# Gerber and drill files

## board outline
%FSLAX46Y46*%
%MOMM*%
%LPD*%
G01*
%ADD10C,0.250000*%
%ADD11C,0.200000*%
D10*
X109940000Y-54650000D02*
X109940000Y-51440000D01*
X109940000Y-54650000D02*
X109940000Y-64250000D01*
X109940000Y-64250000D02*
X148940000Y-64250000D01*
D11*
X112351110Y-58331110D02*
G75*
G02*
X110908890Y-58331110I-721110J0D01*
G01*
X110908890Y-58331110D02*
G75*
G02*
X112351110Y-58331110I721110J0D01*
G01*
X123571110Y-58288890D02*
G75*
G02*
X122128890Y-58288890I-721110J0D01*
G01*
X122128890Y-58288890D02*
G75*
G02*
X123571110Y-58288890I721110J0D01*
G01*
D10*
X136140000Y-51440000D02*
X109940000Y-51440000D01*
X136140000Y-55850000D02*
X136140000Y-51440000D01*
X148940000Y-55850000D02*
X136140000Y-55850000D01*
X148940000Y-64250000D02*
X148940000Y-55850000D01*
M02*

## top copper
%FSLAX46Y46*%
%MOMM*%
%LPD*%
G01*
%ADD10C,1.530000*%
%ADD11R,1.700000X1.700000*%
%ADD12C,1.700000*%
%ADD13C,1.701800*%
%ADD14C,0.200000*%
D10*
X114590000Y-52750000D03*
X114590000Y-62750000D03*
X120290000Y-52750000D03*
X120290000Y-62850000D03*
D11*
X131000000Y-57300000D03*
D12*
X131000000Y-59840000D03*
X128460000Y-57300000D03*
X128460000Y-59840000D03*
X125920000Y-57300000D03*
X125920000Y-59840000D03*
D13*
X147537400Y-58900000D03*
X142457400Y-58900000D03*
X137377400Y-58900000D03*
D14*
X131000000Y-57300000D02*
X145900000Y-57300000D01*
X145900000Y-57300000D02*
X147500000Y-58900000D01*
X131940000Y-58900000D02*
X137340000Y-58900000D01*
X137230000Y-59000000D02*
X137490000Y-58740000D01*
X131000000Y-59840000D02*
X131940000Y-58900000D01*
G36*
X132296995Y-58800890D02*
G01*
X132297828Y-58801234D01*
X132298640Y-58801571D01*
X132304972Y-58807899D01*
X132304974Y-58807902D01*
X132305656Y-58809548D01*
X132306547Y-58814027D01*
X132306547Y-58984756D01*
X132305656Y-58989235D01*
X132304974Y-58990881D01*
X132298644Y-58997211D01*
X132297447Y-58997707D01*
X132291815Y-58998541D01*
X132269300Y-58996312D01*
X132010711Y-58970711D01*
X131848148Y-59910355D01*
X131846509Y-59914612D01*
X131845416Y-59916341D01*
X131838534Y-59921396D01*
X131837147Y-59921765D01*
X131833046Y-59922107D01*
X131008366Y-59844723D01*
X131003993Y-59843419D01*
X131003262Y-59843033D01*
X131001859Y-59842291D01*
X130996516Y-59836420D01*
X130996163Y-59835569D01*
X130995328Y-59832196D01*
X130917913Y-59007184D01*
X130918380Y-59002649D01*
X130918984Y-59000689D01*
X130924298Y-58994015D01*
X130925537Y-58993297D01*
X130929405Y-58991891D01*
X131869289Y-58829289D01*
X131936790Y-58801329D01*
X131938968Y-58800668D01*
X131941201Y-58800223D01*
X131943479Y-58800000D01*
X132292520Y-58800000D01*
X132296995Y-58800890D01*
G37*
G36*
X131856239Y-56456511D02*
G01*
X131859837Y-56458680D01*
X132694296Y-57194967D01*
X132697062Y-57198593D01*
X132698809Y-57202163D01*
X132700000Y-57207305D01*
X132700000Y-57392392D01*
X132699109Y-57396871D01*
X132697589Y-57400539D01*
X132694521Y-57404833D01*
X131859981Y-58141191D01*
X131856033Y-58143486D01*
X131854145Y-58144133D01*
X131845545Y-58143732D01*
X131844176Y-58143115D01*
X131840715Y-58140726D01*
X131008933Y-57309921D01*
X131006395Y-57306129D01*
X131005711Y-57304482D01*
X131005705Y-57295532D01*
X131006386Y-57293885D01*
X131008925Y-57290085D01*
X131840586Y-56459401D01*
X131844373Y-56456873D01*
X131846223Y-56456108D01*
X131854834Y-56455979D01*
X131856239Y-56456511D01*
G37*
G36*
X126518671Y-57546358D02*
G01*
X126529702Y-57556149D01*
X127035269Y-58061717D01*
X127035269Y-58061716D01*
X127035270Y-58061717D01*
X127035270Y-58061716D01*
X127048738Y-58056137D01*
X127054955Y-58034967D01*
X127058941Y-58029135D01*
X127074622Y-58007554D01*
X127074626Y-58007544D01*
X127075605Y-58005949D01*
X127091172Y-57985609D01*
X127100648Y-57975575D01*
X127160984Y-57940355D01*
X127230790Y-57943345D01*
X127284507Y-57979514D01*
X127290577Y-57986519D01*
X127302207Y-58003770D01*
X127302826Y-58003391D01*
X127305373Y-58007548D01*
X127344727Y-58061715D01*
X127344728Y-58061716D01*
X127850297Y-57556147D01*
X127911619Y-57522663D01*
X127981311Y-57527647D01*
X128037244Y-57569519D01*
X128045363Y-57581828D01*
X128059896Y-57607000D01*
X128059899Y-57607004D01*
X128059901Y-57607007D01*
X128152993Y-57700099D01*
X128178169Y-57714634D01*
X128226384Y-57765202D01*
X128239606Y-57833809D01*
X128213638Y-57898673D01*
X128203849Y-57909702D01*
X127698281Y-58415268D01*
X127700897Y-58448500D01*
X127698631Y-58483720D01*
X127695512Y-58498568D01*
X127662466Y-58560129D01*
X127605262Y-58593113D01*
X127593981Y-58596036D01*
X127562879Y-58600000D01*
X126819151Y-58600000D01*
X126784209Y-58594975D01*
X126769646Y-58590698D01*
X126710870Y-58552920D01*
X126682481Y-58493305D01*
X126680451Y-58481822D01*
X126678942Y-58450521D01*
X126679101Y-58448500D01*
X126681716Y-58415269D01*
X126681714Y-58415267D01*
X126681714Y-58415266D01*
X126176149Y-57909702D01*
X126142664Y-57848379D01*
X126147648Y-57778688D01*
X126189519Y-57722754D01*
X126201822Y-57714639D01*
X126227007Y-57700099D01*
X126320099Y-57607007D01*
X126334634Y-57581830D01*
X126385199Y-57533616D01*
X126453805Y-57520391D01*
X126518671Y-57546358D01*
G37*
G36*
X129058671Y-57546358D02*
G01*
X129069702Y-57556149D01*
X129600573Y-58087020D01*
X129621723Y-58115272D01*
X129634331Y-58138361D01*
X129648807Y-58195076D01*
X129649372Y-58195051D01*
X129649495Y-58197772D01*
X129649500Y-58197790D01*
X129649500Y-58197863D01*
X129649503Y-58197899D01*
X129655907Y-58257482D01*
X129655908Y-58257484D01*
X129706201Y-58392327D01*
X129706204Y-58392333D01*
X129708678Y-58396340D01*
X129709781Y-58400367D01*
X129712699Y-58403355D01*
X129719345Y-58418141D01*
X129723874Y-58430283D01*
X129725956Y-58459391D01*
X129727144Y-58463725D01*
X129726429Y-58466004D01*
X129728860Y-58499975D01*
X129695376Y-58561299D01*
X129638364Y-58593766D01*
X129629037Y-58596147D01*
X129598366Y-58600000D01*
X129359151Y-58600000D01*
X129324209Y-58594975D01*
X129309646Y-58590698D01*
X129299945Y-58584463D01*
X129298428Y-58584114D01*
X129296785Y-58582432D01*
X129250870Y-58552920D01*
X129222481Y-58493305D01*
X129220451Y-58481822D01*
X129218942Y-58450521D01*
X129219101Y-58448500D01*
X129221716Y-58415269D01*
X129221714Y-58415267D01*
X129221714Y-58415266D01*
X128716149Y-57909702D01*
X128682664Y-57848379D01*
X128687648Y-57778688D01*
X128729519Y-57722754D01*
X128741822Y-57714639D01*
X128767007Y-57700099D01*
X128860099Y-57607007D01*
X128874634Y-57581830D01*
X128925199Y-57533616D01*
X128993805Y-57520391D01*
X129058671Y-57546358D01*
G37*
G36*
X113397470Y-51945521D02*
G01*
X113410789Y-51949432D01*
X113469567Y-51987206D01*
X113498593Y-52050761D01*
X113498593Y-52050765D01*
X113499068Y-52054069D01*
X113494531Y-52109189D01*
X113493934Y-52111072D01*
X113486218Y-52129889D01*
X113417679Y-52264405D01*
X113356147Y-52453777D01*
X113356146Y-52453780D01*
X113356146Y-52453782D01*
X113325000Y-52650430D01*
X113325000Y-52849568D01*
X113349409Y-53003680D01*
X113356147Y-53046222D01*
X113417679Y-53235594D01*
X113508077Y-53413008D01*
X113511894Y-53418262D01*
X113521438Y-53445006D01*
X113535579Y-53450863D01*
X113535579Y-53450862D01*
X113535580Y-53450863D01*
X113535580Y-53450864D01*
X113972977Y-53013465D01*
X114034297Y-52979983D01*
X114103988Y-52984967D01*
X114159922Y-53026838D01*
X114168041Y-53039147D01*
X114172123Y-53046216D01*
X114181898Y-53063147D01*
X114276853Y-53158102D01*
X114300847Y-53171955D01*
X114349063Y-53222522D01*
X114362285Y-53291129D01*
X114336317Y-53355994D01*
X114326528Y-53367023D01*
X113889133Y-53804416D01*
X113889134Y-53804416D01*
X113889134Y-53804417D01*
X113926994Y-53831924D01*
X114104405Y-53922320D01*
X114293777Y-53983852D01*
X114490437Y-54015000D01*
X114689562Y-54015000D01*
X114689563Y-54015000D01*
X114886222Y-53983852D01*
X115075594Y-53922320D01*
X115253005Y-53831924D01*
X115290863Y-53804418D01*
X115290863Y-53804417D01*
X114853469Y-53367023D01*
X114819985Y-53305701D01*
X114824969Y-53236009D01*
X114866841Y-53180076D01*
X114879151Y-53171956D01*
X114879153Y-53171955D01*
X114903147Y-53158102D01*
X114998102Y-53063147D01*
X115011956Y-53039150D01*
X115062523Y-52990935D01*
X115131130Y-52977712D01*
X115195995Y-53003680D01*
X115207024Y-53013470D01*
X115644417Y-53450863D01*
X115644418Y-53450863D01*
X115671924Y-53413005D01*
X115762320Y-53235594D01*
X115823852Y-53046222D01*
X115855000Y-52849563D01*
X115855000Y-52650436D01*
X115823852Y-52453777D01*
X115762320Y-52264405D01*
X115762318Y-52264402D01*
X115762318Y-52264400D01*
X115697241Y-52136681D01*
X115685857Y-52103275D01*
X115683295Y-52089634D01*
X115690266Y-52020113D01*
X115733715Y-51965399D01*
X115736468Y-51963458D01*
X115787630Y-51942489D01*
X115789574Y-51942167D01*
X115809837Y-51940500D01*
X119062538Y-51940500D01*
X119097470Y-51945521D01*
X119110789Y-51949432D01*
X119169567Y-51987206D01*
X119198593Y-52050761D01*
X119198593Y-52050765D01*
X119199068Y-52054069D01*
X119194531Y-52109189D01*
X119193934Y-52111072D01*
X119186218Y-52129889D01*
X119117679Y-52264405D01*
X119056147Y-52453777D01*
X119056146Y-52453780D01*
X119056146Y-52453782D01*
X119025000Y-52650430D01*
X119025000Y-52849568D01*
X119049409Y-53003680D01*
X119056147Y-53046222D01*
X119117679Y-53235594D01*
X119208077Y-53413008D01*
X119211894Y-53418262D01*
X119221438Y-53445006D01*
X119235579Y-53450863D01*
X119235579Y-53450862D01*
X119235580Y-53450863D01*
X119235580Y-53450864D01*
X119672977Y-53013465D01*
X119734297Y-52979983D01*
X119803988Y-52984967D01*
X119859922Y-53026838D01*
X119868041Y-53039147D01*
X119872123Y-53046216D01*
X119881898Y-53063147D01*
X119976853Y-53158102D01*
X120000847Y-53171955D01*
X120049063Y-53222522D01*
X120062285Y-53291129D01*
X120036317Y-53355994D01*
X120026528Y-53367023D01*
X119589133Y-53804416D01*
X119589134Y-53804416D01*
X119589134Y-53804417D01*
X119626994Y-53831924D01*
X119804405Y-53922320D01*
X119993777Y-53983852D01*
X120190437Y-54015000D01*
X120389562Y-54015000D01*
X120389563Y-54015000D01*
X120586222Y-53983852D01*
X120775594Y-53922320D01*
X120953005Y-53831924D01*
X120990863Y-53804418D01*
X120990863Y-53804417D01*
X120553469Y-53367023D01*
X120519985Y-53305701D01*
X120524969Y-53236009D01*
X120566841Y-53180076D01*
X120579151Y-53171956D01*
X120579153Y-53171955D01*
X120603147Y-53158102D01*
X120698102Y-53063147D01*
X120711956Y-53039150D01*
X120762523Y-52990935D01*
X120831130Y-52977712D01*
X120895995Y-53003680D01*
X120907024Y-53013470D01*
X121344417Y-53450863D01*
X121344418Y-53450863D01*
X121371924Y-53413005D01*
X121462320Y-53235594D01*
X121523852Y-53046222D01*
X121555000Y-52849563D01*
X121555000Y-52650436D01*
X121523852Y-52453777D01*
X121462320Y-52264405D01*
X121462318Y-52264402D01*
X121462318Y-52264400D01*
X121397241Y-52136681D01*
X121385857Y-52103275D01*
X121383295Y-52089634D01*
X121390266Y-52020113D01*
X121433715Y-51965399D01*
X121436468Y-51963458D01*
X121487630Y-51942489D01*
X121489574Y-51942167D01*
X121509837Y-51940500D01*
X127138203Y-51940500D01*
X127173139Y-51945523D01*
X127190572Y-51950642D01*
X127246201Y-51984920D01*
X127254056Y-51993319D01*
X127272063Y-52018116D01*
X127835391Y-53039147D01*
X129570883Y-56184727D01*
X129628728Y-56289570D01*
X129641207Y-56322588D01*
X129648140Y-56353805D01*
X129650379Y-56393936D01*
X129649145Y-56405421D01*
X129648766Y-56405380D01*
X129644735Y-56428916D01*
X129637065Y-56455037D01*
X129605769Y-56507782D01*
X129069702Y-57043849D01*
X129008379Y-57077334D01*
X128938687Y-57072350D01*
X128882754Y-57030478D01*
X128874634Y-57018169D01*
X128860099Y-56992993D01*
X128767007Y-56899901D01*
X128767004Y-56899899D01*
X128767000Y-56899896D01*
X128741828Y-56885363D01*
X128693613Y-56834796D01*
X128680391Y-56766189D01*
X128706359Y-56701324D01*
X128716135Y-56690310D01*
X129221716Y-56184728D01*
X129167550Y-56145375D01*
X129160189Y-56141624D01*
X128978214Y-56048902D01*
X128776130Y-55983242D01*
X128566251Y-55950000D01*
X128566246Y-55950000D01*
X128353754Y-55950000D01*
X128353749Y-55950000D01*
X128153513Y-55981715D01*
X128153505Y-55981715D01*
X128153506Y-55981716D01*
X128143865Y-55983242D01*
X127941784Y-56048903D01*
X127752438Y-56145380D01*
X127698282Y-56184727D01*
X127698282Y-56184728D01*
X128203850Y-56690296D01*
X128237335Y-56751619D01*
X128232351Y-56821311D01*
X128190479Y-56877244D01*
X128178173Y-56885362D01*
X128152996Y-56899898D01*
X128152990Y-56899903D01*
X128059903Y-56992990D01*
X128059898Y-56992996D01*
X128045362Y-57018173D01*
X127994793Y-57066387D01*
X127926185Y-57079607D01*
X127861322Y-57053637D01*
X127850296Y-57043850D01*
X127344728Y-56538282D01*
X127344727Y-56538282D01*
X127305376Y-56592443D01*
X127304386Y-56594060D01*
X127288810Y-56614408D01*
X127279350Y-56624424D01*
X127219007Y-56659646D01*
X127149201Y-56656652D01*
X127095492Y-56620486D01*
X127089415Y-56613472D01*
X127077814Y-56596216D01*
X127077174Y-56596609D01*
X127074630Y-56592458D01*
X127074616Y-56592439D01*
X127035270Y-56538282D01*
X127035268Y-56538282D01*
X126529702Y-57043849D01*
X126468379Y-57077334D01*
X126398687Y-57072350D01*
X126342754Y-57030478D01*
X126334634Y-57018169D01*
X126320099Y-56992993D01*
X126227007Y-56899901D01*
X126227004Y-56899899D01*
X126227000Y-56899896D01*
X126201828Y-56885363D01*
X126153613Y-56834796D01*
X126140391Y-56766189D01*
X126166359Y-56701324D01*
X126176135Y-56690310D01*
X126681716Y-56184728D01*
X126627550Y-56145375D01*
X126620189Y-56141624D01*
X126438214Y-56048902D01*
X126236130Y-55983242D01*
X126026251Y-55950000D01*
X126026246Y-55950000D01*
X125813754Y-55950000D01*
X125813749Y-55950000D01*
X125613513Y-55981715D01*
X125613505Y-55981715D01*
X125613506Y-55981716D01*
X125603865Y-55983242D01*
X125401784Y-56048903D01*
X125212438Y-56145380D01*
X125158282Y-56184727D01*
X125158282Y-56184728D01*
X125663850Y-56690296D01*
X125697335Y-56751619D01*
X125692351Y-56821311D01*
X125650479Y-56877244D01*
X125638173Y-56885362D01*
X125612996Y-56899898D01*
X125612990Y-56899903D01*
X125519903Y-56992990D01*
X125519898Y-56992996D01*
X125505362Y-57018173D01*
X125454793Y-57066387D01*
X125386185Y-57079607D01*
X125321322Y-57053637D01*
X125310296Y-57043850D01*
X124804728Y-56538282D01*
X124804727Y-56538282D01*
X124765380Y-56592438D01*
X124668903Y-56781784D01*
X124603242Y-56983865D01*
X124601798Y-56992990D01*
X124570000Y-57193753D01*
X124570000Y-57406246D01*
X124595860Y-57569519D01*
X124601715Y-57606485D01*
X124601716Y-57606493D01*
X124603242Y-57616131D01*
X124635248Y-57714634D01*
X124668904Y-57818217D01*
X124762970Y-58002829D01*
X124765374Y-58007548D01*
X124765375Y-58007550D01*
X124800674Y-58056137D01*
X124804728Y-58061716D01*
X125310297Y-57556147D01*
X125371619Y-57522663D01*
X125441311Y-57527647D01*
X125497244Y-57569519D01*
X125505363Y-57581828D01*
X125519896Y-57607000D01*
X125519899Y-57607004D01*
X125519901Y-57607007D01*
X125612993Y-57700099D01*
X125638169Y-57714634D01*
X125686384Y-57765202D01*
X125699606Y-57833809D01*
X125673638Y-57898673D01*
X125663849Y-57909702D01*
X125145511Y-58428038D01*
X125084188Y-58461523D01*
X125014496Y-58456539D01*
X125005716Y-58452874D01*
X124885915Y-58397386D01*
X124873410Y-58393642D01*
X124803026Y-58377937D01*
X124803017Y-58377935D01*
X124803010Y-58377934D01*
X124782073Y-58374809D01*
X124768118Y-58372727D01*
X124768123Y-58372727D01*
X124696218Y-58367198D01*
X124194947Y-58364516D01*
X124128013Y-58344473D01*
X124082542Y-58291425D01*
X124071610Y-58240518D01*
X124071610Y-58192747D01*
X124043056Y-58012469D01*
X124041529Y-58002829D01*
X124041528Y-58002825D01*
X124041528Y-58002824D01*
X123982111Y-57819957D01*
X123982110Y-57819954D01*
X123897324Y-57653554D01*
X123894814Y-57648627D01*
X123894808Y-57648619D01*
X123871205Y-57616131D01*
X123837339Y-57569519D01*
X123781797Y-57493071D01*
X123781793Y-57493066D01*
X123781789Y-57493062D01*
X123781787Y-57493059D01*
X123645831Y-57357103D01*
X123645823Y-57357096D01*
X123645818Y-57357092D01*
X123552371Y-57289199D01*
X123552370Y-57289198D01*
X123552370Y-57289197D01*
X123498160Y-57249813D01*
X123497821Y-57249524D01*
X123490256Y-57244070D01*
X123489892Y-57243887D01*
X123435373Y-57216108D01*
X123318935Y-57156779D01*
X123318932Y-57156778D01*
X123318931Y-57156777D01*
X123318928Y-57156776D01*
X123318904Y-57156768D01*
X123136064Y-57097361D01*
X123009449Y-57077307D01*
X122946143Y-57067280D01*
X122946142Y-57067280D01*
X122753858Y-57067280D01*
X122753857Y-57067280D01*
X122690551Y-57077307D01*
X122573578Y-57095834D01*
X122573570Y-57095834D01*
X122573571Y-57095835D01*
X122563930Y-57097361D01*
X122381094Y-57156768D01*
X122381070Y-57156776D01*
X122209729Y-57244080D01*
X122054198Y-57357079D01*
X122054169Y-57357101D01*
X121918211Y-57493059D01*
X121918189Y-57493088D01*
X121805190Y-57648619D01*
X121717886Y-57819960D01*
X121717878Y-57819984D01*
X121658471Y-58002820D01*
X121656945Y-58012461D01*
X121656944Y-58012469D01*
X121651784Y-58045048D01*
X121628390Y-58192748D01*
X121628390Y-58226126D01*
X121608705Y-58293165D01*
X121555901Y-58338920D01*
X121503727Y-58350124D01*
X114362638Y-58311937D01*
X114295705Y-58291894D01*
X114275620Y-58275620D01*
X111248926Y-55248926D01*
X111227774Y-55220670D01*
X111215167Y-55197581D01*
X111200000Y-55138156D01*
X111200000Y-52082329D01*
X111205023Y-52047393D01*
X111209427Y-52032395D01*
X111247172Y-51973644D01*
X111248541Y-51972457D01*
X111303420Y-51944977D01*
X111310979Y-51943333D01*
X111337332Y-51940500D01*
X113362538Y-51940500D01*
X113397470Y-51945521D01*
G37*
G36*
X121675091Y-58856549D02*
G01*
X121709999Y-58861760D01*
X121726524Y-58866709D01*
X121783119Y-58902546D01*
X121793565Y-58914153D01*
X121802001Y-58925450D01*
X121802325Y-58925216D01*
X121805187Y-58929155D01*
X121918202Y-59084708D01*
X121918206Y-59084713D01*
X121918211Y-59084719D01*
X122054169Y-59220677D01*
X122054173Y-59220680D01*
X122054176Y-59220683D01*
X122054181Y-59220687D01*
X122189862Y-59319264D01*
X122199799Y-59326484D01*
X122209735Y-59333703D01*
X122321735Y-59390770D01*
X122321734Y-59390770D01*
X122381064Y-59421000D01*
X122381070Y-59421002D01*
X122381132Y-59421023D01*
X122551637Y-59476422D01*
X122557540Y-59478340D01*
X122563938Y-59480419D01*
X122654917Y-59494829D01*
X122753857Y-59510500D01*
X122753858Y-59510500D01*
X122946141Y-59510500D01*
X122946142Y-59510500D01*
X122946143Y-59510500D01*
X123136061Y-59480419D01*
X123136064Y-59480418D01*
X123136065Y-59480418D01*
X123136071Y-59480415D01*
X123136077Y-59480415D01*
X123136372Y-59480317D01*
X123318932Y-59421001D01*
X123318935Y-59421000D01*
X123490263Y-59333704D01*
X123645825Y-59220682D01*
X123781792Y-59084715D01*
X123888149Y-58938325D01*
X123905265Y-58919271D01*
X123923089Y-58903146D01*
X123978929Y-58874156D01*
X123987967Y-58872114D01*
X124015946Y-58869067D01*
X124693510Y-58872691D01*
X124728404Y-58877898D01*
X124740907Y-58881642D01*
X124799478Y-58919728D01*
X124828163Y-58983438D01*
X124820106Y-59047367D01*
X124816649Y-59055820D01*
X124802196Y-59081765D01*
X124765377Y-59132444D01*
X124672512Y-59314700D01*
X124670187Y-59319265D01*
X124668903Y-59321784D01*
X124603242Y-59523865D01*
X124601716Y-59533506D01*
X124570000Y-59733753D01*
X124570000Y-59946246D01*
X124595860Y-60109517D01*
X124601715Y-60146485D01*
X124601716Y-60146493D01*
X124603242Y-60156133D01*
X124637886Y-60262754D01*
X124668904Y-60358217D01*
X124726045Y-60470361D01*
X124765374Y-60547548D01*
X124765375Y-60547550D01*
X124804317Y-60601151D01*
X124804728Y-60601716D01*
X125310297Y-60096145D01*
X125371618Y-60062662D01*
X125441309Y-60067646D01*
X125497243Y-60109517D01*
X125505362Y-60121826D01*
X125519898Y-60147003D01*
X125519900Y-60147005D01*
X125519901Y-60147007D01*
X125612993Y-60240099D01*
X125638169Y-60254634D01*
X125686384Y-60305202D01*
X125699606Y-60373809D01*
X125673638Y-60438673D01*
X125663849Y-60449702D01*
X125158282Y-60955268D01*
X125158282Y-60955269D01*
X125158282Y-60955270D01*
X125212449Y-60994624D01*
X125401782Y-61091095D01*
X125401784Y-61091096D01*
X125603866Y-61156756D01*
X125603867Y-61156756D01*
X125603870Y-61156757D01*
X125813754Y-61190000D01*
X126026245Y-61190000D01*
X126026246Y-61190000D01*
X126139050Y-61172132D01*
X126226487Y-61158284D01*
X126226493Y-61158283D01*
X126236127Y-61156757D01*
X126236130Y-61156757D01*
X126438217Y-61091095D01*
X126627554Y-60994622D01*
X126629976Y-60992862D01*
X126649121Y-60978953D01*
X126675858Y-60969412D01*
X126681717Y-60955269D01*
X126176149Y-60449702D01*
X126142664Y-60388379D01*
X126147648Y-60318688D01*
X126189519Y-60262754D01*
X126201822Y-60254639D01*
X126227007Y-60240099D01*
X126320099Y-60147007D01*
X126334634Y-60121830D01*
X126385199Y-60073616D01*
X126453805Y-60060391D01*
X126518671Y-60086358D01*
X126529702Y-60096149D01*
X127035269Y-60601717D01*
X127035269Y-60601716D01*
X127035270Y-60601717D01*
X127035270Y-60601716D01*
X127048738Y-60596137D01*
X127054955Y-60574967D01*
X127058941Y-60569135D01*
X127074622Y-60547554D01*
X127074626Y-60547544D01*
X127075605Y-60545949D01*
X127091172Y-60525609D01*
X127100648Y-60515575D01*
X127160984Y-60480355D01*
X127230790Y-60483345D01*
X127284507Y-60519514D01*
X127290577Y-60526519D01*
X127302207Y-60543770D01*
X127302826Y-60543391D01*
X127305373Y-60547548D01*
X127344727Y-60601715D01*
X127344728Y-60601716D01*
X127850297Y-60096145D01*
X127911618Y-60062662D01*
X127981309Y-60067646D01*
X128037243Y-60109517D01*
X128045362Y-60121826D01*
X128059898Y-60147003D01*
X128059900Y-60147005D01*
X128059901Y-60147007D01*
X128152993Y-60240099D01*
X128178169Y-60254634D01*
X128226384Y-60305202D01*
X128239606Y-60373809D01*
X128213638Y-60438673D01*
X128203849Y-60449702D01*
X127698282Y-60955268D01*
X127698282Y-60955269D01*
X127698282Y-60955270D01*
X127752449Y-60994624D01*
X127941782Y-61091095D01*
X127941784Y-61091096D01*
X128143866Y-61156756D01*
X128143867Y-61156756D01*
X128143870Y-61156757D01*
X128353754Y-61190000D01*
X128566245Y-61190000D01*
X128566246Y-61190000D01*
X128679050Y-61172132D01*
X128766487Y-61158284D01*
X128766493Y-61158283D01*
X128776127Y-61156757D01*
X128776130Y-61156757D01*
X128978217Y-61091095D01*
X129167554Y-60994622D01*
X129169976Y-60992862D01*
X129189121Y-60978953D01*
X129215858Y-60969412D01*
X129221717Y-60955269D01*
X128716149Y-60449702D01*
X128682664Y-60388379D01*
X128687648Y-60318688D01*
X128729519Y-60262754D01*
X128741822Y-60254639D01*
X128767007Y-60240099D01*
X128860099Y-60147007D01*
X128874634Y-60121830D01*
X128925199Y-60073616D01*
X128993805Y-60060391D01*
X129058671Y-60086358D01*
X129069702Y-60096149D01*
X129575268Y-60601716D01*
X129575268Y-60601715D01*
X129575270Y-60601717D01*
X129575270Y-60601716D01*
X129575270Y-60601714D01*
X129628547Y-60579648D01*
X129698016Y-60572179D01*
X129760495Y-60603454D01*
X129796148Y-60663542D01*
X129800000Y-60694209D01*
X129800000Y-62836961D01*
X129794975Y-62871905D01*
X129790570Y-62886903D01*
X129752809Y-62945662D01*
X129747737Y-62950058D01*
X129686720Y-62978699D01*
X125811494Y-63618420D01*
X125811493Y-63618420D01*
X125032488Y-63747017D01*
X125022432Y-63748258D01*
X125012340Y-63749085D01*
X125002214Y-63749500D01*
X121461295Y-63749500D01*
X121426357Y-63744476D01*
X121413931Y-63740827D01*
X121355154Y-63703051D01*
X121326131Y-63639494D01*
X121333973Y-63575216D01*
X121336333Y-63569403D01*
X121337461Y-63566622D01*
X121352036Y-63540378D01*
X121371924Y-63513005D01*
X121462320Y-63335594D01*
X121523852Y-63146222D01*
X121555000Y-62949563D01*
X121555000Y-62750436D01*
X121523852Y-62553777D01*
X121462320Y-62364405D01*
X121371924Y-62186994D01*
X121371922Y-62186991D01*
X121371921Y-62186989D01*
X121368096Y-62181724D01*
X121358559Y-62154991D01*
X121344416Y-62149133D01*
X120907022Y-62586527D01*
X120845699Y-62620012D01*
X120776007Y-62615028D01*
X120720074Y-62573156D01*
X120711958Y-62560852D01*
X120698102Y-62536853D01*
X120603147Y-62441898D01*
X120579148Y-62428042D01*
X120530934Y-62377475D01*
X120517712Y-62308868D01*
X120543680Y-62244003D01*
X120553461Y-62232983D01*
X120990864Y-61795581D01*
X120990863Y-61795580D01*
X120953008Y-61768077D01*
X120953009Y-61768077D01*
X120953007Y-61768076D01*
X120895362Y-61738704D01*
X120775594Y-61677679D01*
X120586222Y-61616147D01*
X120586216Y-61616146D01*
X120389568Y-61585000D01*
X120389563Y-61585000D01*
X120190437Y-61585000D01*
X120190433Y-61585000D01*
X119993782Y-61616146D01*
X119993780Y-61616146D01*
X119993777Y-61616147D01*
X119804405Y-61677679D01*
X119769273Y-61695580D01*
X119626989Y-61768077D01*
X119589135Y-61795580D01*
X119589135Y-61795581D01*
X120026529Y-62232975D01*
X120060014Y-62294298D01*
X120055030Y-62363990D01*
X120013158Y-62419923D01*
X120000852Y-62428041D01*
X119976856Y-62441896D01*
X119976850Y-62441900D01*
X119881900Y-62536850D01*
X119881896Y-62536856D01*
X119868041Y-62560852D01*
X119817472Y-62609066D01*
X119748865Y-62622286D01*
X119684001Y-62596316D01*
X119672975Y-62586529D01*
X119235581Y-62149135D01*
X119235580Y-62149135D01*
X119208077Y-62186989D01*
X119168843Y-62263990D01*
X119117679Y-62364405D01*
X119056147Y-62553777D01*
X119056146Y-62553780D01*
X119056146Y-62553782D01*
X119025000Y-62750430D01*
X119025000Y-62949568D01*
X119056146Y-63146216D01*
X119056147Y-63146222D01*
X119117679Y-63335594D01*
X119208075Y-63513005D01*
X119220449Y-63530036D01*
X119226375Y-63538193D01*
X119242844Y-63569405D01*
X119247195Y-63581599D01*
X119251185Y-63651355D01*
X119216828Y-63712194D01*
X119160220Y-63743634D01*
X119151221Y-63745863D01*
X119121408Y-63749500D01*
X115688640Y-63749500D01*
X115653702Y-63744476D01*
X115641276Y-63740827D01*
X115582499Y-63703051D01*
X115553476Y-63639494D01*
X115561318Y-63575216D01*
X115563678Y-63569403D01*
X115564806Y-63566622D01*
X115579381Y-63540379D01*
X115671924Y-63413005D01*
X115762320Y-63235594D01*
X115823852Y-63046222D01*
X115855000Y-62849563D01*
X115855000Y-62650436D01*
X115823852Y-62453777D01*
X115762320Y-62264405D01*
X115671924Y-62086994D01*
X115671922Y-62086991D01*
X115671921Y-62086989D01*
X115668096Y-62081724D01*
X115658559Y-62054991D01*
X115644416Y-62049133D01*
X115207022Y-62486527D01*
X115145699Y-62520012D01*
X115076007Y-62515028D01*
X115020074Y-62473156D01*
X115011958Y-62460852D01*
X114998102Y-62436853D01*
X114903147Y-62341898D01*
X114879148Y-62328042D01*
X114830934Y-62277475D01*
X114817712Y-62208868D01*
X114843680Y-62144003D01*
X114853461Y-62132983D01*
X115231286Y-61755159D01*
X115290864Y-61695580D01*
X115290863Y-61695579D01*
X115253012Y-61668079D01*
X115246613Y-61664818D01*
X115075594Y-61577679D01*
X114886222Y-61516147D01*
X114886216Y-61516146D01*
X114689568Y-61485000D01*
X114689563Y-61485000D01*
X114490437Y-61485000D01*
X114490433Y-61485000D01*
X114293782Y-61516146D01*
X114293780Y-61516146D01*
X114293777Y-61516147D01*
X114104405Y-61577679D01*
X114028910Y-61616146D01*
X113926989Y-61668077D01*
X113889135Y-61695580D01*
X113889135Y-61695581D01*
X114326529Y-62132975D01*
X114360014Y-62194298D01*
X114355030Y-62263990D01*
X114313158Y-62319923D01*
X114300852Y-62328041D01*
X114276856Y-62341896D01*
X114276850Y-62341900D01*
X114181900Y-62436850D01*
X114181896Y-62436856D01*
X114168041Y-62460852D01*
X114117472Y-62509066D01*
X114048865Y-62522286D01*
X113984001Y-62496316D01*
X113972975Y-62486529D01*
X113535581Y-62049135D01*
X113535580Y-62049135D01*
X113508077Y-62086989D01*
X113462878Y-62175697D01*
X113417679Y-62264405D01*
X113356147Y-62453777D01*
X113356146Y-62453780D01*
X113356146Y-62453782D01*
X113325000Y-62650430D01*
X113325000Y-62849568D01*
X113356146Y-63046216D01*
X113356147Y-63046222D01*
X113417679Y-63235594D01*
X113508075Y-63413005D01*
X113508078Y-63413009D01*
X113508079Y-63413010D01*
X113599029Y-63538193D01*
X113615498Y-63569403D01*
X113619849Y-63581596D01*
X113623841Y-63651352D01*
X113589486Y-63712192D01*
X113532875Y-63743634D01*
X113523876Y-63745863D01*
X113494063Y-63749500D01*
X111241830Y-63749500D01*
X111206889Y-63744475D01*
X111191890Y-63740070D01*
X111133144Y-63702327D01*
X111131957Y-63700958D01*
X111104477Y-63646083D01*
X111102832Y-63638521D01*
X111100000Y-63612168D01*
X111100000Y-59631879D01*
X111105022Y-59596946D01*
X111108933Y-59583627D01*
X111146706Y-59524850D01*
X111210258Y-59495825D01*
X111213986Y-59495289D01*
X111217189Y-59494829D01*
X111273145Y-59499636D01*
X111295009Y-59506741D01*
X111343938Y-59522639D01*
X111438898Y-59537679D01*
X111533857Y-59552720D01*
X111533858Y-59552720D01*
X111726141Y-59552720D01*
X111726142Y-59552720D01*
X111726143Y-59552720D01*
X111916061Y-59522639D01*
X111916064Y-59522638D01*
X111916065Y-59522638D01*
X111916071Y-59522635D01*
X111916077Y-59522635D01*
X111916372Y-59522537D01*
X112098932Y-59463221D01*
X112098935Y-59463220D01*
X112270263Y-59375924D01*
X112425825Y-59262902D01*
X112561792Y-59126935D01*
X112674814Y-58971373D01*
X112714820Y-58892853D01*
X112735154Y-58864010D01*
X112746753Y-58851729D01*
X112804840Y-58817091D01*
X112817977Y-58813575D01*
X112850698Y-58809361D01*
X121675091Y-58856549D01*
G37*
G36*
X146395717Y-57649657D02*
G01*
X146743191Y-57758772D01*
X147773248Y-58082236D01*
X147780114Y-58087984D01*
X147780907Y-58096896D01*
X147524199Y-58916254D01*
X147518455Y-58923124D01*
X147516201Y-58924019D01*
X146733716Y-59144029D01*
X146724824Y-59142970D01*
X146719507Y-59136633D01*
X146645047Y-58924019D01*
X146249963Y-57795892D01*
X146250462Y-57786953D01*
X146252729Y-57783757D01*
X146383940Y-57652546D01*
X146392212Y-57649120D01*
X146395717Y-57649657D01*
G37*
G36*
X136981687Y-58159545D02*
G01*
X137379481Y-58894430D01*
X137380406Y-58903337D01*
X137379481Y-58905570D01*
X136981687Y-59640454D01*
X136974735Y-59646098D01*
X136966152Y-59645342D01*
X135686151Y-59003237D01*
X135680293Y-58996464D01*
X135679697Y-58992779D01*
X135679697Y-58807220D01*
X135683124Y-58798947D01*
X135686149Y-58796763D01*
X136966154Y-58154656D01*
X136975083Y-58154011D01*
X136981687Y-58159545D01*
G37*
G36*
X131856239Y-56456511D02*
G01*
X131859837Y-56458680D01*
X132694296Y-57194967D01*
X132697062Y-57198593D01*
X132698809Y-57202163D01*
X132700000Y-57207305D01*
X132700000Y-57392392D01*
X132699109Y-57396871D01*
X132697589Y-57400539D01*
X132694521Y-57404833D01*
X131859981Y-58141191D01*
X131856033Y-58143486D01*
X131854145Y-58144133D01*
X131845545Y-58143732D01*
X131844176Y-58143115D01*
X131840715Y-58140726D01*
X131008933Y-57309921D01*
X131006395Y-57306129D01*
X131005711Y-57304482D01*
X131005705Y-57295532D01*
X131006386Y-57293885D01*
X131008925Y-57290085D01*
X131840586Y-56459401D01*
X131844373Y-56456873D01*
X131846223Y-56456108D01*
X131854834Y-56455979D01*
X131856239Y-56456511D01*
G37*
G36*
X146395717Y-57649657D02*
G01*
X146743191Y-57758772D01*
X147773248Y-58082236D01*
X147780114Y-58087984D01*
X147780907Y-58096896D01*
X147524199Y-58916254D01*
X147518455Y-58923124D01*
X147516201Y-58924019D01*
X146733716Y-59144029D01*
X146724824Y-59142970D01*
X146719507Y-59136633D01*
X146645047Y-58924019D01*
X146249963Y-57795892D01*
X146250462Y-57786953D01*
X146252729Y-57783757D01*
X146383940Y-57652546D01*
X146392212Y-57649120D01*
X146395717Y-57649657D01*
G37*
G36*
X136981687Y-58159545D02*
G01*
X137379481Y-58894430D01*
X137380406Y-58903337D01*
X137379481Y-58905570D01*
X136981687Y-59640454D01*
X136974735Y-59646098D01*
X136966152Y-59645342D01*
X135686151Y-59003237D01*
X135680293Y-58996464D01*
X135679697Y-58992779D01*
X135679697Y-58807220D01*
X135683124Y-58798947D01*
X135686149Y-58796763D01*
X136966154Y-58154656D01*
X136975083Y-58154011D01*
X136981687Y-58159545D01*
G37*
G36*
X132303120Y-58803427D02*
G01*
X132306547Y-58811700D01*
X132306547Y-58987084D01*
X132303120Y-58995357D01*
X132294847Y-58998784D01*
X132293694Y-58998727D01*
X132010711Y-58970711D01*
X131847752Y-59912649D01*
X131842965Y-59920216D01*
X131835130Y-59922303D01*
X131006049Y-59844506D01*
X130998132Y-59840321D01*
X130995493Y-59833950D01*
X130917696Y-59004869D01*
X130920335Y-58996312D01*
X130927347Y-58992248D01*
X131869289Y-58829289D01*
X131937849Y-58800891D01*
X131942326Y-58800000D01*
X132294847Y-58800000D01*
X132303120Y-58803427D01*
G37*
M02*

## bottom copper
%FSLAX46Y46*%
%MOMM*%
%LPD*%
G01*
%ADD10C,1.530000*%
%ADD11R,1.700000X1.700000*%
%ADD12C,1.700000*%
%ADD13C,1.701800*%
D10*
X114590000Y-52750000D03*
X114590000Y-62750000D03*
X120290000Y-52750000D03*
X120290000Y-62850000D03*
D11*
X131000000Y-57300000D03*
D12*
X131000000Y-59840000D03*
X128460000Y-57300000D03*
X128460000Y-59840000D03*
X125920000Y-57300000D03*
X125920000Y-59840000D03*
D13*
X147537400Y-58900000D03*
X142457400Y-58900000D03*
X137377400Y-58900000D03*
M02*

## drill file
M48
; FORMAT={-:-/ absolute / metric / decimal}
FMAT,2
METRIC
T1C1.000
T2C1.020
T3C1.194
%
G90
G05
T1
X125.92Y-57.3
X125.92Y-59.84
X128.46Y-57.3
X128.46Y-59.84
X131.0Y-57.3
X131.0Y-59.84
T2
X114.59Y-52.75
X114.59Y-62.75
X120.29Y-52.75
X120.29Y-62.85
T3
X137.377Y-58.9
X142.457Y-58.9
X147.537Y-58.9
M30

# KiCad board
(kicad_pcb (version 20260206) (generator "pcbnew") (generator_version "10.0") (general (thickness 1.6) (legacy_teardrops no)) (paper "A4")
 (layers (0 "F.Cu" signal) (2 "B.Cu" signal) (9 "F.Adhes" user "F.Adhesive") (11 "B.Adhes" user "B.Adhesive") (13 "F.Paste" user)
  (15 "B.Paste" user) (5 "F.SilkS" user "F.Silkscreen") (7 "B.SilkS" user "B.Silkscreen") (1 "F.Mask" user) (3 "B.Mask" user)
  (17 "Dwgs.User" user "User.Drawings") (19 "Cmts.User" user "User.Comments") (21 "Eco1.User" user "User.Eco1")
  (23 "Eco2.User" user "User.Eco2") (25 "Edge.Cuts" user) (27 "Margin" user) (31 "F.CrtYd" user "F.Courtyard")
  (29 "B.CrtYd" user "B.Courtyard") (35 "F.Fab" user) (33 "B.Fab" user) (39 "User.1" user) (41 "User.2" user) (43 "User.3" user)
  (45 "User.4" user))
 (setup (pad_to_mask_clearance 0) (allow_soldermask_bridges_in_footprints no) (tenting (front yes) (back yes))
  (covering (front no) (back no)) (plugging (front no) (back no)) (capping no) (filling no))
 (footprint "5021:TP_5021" (layer "F.Cu") (at 114.59 52.75 -90)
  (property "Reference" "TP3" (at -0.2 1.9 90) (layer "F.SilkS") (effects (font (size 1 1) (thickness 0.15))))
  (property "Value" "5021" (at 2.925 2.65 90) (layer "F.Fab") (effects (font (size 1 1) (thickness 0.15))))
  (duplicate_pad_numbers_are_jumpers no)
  (pad "TP" thru_hole circle (at 0 0 270) (size 1.53 1.53) (drill 1.02) (layers "*.Cu" "*.Mask") (remove_unused_layers no)
   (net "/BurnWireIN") (solder_mask_margin 0.102)
   (teardrops (best_length_ratio 0.5) (max_length 1) (best_width_ratio 1) (max_width 2) (curved_edges no) (filter_ratio 0.9) (enabled yes)
    (allow_two_segments yes) (prefer_zone_connections yes))))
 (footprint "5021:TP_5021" (layer "F.Cu") (at 114.59 62.75 -90)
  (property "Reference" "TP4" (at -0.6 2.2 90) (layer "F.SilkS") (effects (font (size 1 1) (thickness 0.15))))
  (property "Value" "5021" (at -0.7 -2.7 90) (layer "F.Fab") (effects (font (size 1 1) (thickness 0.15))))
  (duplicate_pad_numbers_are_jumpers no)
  (pad "TP" thru_hole circle (at 0 0 270) (size 1.53 1.53) (drill 1.02) (layers "*.Cu" "*.Mask") (remove_unused_layers no) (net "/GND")
   (solder_mask_margin 0.102)
   (teardrops (best_length_ratio 0.5) (max_length 1) (best_width_ratio 1) (max_width 2) (curved_edges no) (filter_ratio 0.9) (enabled yes)
    (allow_two_segments yes) (prefer_zone_connections yes))))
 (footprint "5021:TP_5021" (layer "F.Cu") (at 120.29 52.75 -90)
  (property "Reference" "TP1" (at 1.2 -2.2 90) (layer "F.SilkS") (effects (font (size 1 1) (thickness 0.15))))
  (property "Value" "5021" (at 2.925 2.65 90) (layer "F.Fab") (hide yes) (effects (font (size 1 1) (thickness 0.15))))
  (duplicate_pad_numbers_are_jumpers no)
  (pad "TP" thru_hole circle (at 0 0 270) (size 1.53 1.53) (drill 1.02) (layers "*.Cu" "*.Mask") (remove_unused_layers no)
   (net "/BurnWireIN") (solder_mask_margin 0.102)
   (teardrops (best_length_ratio 0.5) (max_length 1) (best_width_ratio 1) (max_width 2) (curved_edges no) (filter_ratio 0.9) (enabled yes)
    (allow_two_segments yes) (prefer_zone_connections yes))))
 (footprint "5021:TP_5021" (layer "F.Cu") (at 120.29 62.85 -90)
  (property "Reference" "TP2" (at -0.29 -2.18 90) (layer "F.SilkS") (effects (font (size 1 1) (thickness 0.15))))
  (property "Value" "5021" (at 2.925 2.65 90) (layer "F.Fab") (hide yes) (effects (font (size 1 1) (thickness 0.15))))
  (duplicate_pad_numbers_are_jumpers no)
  (pad "TP" thru_hole circle (at 0 0 270) (size 1.53 1.53) (drill 1.02) (layers "*.Cu" "*.Mask") (remove_unused_layers no) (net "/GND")
   (solder_mask_margin 0.102)
   (teardrops (best_length_ratio 0.5) (max_length 1) (best_width_ratio 1) (max_width 2) (curved_edges no) (filter_ratio 0.9) (enabled yes)
    (allow_two_segments yes) (prefer_zone_connections yes))))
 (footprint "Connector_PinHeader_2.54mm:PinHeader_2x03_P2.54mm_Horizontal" (layer "F.Cu") (at 131 57.3 -90)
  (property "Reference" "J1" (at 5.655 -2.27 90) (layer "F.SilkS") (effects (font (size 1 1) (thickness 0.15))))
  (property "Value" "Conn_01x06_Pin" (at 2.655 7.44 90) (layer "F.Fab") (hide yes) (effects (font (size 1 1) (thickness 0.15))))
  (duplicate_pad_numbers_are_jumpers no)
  (pad "1" thru_hole rect (at 0 0 270) (size 1.7 1.7) (drill 1) (layers "*.Cu" "*.Mask") (remove_unused_layers no)
   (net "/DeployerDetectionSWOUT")
   (teardrops (best_length_ratio 0.5) (max_length 1) (best_width_ratio 1) (max_width 2) (curved_edges no) (filter_ratio 0.9) (enabled yes)
    (allow_two_segments yes) (prefer_zone_connections yes)))
  (pad "2" thru_hole circle (at 2.54 0 270) (size 1.7 1.7) (drill 1) (layers "*.Cu" "*.Mask") (remove_unused_layers no)
   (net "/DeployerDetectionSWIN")
   (teardrops (best_length_ratio 0.5) (max_length 1) (best_width_ratio 1) (max_width 2) (curved_edges no) (filter_ratio 0.9) (enabled yes)
    (allow_two_segments yes) (prefer_zone_connections yes)))
  (pad "3" thru_hole circle (at 0 2.54 270) (size 1.7 1.7) (drill 1) (layers "*.Cu" "*.Mask") (remove_unused_layers no) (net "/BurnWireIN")
   (teardrops (best_length_ratio 0.5) (max_length 1) (best_width_ratio 1) (max_width 2) (curved_edges no) (filter_ratio 0.9) (enabled yes)
    (allow_two_segments yes) (prefer_zone_connections yes)))
  (pad "4" thru_hole circle (at 2.54 2.54 270) (size 1.7 1.7) (drill 1) (layers "*.Cu" "*.Mask") (remove_unused_layers no) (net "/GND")
   (teardrops (best_length_ratio 0.5) (max_length 1) (best_width_ratio 1) (max_width 2) (curved_edges no) (filter_ratio 0.9) (enabled yes)
    (allow_two_segments yes) (prefer_zone_connections yes)))
  (pad "5" thru_hole circle (at 0 5.08 270) (size 1.7 1.7) (drill 1) (layers "*.Cu" "*.Mask") (remove_unused_layers no) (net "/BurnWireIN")
   (teardrops (best_length_ratio 0.5) (max_length 1) (best_width_ratio 1) (max_width 2) (curved_edges no) (filter_ratio 0.9) (enabled yes)
    (allow_two_segments yes) (prefer_zone_connections yes)))
  (pad "6" thru_hole circle (at 2.54 5.08 270) (size 1.7 1.7) (drill 1) (layers "*.Cu" "*.Mask") (remove_unused_layers no) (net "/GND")
   (teardrops (best_length_ratio 0.5) (max_length 1) (best_width_ratio 1) (max_width 2) (curved_edges no) (filter_ratio 0.9) (enabled yes)
    (allow_two_segments yes) (prefer_zone_connections yes))))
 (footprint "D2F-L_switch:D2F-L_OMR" (layer "B.Cu") (at 147.5374 58.9 180)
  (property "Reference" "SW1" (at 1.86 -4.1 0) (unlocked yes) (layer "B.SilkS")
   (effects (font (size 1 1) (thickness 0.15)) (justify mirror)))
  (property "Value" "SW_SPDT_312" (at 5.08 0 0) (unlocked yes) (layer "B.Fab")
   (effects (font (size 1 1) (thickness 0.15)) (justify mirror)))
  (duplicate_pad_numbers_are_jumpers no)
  (pad "1" thru_hole circle (at 0 0 180) (size 1.7018 1.7018) (drill 1.1938) (layers "*.Cu" "*.Mask") (remove_unused_layers no)
   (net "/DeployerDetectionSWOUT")
   (teardrops (best_length_ratio 0.5) (max_length 1) (best_width_ratio 1) (max_width 2) (curved_edges no) (filter_ratio 0.9) (enabled yes)
    (allow_two_segments yes) (prefer_zone_connections yes)))
  (pad "2" thru_hole circle (at 5.08 0 180) (size 1.7018 1.7018) (drill 1.1938) (layers "*.Cu" "*.Mask") (remove_unused_layers no)
   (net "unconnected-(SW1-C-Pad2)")
   (teardrops (best_length_ratio 0.5) (max_length 1) (best_width_ratio 1) (max_width 2) (curved_edges no) (filter_ratio 0.9) (enabled yes)
    (allow_two_segments yes) (prefer_zone_connections yes)))
  (pad "3" thru_hole circle (at 10.16 0 180) (size 1.7018 1.7018) (drill 1.1938) (layers "*.Cu" "*.Mask") (remove_unused_layers no)
   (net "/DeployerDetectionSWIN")
   (teardrops (best_length_ratio 0.5) (max_length 1) (best_width_ratio 1) (max_width 2) (curved_edges no) (filter_ratio 0.9) (enabled yes)
    (allow_two_segments yes) (prefer_zone_connections yes))))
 (gr_line (start 109.94 54.65) (end 109.94 51.44) (stroke (width 0.25) (type solid)) (layer "Edge.Cuts"))
 (gr_line (start 109.94 54.65) (end 109.94 64.25) (stroke (width 0.25) (type default)) (layer "Edge.Cuts"))
 (gr_line (start 109.94 64.25) (end 148.94 64.25) (stroke (width 0.25) (type solid)) (layer "Edge.Cuts"))
 (gr_circle (center 111.63 58.33111) (end 112.23 58.73111) (stroke (width 0.2) (type solid)) (fill no) (layer "Edge.Cuts"))
 (gr_circle (center 122.85 58.28889) (end 123.45 58.68889) (stroke (width 0.2) (type solid)) (fill no) (layer "Edge.Cuts"))
 (gr_line (start 136.14 51.44) (end 109.94 51.44) (stroke (width 0.25) (type default)) (layer "Edge.Cuts"))
 (gr_line (start 136.14 55.85) (end 136.14 51.44) (stroke (width 0.25) (type solid)) (layer "Edge.Cuts"))
 (gr_line (start 148.94 55.85) (end 136.14 55.85) (stroke (width 0.25) (type default)) (layer "Edge.Cuts"))
 (gr_line (start 148.94 64.25) (end 148.94 55.85) (stroke (width 0.25) (type default)) (layer "Edge.Cuts"))
 (segment (start 131 57.3) (end 145.9 57.3) (width 0.2) (layer "F.Cu") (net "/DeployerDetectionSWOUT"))
 (segment (start 145.9 57.3) (end 147.5 58.9) (width 0.2) (layer "F.Cu") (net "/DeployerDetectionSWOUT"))
 (segment (start 131.94 58.9) (end 137.34 58.9) (width 0.2) (layer "F.Cu") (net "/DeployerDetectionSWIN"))
 (segment (start 137.23 59) (end 137.49 58.74) (width 0.2) (layer "F.Cu") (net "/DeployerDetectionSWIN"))
 (segment (start 131 59.84) (end 131.94 58.9) (width 0.2) (layer "F.Cu") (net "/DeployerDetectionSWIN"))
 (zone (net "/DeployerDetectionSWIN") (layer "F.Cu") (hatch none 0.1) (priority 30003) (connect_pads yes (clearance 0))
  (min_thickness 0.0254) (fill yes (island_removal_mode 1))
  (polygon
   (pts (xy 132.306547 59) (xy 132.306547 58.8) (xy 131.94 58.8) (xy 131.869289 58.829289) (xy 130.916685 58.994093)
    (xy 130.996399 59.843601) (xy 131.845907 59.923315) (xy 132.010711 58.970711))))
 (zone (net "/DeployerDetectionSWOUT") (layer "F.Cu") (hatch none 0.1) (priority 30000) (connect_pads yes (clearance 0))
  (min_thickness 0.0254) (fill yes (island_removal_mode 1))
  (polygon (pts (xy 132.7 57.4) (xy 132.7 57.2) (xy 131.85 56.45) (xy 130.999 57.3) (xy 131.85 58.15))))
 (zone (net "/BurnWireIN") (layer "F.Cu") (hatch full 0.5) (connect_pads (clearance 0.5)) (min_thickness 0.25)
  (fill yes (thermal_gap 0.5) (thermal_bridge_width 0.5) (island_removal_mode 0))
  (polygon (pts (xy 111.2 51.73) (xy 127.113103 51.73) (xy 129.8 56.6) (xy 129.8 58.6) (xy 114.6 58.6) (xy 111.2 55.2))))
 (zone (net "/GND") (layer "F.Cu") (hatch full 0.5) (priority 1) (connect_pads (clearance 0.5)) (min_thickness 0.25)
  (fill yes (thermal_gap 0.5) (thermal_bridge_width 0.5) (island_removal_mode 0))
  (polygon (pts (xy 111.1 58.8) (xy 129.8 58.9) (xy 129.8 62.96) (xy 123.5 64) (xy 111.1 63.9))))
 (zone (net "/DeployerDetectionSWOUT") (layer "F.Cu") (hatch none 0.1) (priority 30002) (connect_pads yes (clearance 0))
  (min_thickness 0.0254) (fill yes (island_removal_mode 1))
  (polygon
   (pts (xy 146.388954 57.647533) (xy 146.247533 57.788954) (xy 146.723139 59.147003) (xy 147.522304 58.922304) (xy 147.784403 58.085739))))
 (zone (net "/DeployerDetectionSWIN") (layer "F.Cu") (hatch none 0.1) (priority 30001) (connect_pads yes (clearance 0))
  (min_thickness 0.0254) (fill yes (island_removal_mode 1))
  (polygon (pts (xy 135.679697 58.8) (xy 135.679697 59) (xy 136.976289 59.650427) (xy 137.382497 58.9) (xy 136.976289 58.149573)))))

